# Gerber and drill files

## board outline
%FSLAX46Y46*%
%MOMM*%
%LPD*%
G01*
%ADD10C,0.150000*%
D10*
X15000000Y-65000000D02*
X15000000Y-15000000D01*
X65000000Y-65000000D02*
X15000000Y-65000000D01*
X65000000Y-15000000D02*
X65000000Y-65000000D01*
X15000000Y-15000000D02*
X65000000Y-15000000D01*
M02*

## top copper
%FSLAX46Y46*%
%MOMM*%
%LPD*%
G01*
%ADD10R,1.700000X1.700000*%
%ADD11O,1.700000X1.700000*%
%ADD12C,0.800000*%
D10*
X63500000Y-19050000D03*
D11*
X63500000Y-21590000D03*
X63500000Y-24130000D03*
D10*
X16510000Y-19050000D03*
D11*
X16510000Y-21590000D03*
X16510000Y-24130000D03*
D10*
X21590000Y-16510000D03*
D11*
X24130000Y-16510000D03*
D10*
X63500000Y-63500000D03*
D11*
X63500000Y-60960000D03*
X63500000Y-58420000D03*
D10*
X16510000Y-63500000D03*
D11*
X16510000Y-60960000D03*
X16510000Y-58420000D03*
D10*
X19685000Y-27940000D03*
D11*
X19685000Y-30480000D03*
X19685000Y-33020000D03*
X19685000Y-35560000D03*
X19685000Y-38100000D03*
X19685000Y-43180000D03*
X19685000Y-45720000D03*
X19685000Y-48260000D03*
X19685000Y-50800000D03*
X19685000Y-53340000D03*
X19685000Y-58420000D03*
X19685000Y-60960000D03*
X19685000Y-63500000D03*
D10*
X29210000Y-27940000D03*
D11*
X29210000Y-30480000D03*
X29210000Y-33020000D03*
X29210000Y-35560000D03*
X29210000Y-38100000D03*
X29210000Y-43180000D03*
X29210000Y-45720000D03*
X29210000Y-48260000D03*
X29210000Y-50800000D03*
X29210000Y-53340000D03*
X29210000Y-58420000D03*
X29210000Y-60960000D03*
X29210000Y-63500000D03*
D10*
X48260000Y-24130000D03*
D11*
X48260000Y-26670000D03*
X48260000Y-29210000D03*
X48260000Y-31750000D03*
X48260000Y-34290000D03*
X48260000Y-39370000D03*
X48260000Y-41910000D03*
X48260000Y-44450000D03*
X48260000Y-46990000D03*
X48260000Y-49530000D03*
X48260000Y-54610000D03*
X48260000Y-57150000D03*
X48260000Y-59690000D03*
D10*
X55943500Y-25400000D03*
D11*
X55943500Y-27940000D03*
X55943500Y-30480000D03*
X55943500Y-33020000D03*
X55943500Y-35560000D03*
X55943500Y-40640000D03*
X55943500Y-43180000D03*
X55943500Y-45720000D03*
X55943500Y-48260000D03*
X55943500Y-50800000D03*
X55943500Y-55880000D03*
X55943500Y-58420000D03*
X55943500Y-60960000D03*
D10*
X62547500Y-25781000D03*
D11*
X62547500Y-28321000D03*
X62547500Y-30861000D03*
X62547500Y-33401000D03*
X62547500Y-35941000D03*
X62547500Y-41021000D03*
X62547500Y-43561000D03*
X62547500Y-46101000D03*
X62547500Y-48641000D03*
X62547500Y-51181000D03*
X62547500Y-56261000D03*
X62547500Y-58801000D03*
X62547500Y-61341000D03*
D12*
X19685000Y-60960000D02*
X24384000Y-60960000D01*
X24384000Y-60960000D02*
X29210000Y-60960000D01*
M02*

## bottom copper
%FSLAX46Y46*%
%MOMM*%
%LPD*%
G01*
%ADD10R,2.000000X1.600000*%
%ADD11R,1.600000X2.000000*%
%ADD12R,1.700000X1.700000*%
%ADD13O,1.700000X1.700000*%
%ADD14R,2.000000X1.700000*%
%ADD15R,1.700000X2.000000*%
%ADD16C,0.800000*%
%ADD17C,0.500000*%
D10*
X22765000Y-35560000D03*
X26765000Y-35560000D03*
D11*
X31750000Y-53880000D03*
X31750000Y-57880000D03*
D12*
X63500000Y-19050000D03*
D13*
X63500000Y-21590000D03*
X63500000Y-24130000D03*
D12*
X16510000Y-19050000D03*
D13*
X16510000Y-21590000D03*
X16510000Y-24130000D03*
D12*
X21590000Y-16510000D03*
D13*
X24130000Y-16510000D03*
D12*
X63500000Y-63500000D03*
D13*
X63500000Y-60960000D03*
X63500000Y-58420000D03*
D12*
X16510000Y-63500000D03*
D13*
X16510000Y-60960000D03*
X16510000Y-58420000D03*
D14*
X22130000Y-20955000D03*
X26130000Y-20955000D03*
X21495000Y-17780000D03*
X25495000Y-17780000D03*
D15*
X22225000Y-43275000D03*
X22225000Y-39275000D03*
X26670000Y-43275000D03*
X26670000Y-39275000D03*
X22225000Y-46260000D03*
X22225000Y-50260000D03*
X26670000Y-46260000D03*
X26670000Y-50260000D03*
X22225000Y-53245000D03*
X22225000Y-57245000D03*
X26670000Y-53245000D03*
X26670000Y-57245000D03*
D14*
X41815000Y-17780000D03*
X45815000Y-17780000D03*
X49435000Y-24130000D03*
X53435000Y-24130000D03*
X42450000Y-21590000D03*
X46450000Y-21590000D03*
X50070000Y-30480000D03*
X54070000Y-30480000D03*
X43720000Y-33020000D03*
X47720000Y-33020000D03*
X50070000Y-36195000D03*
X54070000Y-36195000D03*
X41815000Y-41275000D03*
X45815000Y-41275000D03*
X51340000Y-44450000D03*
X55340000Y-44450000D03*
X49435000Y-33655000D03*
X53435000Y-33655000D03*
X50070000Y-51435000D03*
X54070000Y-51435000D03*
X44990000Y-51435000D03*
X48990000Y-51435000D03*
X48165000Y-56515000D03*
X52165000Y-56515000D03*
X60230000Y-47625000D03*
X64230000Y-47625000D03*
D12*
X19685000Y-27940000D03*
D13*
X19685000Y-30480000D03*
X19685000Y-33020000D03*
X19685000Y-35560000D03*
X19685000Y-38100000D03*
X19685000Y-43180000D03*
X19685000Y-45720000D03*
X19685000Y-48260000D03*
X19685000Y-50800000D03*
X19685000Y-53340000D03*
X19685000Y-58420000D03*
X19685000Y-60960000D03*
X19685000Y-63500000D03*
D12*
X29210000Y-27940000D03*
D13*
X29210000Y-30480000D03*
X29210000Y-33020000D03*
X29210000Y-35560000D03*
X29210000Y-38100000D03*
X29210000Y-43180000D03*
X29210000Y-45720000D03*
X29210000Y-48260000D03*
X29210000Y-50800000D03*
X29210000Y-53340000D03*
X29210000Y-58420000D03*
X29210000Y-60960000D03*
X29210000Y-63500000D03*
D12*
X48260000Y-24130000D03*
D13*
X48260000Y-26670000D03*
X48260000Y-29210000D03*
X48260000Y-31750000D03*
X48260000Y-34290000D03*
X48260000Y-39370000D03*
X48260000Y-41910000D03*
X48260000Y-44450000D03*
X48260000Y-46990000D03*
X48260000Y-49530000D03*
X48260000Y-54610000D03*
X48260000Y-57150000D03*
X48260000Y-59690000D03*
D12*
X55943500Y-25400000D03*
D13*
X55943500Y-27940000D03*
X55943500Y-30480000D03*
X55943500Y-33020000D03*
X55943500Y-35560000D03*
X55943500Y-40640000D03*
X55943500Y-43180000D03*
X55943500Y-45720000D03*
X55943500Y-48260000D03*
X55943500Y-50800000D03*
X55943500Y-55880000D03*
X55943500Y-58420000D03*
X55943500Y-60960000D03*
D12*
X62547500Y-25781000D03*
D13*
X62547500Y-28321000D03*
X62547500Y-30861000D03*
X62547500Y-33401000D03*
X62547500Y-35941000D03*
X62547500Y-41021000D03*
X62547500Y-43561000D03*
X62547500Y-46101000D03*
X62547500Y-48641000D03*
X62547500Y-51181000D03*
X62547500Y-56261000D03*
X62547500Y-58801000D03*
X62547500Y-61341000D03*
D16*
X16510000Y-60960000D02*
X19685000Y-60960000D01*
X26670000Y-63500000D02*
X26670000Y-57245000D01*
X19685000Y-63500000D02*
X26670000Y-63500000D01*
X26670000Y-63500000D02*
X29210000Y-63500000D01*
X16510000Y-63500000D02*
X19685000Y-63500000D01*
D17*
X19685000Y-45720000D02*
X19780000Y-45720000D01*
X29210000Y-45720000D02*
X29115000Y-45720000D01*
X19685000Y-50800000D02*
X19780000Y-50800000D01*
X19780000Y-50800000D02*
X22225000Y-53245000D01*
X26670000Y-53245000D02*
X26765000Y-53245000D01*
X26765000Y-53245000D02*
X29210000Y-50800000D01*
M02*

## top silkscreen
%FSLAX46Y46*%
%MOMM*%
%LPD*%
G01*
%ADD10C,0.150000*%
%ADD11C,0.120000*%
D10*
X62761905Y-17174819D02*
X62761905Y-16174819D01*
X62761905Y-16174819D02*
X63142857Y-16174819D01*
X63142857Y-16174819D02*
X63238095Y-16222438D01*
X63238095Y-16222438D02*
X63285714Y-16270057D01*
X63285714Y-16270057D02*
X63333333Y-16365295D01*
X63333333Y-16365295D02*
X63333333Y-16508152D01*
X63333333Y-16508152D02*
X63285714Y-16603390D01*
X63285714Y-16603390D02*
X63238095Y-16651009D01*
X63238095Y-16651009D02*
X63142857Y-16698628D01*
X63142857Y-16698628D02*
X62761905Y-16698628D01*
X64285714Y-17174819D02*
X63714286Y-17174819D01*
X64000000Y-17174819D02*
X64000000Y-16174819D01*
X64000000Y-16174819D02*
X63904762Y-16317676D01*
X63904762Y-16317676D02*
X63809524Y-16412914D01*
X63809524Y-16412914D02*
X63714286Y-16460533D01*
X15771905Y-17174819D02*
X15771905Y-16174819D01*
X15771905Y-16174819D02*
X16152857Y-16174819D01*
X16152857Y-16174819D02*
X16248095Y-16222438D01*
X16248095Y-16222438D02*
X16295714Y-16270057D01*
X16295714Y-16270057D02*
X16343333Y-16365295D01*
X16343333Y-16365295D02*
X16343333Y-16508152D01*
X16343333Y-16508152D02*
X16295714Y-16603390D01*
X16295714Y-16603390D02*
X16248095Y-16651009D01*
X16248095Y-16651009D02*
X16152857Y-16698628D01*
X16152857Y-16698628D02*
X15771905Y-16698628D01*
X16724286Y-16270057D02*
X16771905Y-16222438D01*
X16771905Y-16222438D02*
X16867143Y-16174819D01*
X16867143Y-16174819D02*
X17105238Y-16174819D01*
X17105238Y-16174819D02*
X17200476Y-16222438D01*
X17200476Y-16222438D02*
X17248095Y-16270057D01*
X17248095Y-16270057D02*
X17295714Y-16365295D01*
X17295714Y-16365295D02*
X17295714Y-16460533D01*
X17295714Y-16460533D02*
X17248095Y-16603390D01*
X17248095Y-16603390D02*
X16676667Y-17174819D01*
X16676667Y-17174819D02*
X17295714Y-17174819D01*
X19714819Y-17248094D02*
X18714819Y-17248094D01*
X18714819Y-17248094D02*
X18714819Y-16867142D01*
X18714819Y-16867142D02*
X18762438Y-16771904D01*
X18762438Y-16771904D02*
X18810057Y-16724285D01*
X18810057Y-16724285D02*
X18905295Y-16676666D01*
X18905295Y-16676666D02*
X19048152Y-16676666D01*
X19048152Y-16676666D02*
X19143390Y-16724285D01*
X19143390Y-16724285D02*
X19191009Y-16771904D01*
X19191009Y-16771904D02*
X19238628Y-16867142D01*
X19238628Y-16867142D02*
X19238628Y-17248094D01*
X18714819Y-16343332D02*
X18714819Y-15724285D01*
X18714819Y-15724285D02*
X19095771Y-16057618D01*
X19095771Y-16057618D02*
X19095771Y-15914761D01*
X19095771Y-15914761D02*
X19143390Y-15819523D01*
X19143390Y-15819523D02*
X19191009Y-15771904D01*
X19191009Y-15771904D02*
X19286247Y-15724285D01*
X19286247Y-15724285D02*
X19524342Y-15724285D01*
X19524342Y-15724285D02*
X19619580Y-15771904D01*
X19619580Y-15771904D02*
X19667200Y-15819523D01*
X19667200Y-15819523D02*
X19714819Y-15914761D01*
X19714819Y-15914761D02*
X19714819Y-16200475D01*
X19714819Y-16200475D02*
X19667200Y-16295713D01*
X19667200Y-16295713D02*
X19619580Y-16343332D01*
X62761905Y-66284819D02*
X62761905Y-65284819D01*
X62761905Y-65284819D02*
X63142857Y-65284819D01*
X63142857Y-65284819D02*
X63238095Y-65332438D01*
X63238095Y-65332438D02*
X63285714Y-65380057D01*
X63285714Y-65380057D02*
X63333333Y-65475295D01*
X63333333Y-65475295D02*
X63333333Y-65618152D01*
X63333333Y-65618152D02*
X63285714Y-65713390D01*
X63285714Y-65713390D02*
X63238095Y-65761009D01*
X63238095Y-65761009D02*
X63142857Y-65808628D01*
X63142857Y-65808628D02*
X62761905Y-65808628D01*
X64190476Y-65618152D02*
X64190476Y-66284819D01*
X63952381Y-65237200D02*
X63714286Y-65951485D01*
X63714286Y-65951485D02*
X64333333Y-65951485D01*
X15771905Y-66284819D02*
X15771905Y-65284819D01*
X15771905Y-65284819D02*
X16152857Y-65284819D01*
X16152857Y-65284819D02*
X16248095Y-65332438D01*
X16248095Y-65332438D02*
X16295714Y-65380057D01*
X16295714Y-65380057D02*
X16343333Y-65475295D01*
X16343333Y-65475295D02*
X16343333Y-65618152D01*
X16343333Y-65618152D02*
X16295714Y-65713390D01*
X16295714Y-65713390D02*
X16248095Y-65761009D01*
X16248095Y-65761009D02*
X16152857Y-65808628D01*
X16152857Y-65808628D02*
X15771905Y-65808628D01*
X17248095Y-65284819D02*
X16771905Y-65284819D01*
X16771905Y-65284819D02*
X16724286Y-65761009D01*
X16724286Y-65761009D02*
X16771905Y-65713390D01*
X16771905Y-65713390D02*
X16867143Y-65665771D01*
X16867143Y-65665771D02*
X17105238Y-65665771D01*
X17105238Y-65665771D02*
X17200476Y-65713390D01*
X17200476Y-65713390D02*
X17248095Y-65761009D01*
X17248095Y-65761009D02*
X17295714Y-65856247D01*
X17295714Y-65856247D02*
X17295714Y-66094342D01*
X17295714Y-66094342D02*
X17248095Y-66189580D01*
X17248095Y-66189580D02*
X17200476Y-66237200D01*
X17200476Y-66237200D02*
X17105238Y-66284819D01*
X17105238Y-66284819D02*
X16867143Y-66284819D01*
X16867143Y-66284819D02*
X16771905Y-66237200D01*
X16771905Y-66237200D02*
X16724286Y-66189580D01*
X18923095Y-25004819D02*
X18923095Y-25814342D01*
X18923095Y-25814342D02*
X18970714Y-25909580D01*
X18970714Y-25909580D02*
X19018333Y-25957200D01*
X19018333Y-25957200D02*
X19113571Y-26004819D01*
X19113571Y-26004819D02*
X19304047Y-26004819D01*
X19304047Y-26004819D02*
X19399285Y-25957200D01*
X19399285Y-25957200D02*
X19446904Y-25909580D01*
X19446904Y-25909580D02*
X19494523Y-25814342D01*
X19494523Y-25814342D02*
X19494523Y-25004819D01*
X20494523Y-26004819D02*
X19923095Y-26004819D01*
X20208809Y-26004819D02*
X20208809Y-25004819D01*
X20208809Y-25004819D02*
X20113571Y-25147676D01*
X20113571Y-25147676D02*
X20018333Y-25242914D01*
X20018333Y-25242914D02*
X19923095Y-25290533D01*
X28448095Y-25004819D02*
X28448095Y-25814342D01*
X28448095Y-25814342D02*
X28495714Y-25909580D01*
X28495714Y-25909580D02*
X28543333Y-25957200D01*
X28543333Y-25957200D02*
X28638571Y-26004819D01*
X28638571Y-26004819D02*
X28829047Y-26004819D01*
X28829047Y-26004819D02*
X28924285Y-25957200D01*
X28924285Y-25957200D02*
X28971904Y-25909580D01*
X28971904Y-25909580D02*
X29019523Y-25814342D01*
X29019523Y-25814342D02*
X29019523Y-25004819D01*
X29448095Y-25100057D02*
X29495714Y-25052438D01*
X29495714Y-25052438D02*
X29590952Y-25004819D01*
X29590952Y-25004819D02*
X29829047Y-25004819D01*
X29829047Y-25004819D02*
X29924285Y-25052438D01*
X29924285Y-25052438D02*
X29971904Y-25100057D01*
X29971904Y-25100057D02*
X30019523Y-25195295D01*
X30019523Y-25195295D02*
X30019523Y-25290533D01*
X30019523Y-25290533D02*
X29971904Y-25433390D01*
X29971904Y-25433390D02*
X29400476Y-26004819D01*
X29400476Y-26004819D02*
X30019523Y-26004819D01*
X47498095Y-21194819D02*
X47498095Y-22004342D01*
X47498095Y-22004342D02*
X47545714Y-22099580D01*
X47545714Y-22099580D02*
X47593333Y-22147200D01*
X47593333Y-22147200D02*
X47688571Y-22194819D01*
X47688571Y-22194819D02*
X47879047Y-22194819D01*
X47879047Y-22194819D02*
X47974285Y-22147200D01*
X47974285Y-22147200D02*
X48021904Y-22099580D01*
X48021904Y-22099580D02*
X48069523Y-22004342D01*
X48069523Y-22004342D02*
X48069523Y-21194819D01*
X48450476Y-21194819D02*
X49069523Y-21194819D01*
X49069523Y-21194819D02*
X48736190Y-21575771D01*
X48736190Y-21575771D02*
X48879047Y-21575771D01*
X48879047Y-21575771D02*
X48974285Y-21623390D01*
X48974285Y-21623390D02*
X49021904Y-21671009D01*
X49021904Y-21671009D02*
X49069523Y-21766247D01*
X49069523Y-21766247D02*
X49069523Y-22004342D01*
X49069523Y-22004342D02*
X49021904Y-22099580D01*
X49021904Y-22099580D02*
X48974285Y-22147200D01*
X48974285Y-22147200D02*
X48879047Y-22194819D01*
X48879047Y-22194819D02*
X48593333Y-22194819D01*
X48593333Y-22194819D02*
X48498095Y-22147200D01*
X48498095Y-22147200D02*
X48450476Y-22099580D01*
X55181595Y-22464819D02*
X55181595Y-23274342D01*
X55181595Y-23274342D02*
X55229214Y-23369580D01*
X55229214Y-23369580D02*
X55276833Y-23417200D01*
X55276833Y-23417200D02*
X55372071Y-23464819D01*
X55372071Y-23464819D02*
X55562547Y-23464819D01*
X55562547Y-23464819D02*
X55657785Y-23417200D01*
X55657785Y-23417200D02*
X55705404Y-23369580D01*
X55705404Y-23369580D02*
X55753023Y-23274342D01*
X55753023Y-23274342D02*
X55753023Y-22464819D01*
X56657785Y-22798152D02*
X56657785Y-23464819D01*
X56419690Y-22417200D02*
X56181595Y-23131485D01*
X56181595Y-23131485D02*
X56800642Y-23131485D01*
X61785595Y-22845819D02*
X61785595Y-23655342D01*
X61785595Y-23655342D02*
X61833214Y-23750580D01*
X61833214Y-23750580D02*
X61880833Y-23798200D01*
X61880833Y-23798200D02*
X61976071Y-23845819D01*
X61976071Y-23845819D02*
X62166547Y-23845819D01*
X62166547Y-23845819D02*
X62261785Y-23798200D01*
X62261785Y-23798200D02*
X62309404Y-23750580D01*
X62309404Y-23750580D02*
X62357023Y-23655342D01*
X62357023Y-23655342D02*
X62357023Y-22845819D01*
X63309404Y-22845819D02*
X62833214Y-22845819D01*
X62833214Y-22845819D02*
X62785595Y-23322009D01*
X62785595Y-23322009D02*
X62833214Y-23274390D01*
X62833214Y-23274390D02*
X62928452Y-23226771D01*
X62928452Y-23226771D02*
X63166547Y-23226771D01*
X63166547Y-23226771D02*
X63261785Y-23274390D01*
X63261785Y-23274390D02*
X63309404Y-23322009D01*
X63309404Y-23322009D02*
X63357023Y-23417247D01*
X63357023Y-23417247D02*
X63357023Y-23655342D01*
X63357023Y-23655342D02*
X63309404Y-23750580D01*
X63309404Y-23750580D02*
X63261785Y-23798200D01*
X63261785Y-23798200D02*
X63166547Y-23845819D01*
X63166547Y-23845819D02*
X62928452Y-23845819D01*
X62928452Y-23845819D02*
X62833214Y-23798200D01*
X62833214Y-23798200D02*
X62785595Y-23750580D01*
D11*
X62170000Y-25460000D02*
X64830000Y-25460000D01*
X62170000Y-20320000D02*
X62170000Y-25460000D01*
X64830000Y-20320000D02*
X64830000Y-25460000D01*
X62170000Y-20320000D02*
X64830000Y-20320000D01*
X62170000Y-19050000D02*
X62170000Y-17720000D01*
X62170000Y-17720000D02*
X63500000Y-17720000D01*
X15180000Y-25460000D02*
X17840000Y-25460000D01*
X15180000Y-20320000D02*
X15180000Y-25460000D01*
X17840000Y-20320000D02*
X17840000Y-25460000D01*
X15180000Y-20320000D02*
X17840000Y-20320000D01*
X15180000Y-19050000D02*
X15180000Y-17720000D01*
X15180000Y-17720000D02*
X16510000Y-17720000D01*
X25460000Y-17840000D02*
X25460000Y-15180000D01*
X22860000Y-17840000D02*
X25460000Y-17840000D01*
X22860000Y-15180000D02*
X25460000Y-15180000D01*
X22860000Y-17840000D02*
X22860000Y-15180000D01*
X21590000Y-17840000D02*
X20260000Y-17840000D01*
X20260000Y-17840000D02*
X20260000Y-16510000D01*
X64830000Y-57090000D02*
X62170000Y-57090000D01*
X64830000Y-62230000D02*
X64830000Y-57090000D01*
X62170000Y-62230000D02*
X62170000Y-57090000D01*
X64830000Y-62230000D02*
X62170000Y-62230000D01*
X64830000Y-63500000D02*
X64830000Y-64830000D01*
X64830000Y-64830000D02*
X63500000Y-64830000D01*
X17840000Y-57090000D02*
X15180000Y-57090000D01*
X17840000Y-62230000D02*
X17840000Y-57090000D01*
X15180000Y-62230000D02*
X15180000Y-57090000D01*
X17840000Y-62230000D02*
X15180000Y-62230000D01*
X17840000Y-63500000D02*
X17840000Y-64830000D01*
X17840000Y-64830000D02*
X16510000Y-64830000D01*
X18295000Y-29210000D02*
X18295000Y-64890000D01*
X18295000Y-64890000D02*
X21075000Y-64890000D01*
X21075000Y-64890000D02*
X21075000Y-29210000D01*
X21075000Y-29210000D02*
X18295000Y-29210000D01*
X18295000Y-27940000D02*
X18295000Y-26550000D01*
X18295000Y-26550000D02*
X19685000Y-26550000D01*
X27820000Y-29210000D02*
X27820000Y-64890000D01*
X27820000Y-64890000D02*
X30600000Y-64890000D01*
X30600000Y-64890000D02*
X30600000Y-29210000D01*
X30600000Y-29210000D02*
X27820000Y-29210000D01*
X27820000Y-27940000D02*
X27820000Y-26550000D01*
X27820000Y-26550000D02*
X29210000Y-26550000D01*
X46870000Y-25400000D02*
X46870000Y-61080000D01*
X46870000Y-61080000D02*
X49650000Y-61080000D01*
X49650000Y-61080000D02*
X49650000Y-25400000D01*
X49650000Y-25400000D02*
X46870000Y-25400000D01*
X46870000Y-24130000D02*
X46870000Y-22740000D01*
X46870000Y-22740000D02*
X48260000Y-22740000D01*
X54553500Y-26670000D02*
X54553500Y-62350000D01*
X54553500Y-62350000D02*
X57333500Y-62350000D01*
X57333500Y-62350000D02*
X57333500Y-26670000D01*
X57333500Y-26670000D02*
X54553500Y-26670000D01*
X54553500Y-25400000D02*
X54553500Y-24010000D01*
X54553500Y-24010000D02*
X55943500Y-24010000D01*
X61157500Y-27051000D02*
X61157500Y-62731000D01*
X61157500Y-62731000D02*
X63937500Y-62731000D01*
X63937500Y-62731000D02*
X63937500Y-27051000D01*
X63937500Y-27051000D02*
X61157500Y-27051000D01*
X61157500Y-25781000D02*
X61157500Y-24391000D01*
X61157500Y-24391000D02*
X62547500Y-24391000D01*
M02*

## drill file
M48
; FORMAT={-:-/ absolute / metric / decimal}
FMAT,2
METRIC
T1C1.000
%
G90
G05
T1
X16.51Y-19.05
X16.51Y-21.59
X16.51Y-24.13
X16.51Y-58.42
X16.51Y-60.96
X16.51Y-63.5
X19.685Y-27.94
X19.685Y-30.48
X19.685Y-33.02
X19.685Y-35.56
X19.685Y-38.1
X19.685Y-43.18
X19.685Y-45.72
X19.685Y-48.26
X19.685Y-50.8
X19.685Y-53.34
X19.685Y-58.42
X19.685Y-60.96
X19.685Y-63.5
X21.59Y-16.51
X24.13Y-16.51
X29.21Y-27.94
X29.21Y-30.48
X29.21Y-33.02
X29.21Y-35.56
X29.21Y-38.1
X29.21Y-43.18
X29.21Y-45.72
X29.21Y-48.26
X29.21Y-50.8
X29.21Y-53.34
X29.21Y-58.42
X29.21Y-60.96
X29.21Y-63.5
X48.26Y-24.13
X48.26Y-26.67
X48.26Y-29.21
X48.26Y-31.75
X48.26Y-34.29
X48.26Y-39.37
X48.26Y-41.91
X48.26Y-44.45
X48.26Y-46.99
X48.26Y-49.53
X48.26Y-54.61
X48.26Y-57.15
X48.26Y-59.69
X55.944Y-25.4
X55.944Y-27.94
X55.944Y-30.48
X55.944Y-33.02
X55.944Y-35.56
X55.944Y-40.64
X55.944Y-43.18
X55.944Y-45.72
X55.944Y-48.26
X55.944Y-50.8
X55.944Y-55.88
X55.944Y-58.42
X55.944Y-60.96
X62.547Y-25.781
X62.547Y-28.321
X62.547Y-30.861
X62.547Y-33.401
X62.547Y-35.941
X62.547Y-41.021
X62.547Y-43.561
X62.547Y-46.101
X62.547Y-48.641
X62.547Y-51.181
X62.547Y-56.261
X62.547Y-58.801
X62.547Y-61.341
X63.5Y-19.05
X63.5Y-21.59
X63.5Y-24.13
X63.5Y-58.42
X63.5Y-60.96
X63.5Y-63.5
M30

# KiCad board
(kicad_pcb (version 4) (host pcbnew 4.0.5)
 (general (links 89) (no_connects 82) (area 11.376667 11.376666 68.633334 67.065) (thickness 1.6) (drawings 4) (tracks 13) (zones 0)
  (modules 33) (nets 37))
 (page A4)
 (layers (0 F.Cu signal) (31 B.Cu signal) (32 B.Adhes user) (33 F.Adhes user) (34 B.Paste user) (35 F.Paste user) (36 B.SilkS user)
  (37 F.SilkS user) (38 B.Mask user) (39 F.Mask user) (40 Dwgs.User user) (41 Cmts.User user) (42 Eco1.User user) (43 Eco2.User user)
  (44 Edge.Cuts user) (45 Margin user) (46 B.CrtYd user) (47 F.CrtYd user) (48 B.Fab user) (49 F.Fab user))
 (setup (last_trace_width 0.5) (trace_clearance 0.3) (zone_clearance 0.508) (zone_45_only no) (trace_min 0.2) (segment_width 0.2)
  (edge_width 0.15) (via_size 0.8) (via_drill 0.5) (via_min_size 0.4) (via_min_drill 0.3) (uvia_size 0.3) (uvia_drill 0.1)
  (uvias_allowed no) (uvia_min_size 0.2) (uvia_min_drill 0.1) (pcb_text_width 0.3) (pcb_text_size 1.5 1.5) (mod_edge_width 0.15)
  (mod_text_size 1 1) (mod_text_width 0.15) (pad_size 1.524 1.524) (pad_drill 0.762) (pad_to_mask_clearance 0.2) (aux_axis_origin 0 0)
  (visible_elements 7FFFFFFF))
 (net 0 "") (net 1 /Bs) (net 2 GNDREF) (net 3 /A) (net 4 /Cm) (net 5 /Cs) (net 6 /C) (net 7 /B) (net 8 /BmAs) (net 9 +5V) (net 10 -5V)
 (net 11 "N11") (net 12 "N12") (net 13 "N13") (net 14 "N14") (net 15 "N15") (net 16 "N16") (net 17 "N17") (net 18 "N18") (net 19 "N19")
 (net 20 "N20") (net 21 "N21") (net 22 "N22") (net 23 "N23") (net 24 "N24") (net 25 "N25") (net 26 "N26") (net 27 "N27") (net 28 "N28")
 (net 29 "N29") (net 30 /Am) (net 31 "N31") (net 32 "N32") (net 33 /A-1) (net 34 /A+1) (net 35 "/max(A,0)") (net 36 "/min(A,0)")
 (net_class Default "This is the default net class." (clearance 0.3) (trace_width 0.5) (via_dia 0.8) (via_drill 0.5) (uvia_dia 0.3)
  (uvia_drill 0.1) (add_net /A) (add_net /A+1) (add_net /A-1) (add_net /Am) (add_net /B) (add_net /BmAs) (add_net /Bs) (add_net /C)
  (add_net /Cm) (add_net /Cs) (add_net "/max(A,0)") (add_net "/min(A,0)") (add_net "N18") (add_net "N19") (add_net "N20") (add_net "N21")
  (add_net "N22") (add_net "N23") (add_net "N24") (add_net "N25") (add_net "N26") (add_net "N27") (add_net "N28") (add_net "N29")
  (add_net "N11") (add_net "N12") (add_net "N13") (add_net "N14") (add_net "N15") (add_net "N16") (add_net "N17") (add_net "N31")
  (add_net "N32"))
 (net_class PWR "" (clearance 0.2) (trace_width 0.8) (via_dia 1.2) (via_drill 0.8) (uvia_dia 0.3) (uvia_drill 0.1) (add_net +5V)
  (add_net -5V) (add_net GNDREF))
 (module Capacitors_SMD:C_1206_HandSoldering (layer B.Cu) (at 24.765 35.56)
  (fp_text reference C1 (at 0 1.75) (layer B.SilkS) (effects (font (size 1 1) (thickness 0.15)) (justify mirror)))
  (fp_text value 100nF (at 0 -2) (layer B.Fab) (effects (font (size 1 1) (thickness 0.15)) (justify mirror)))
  (pad 1 smd rect (at -2 0) (size 2 1.6) (layers B.Cu B.Paste B.Mask) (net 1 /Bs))
  (pad 2 smd rect (at 2 0) (size 2 1.6) (layers B.Cu B.Paste B.Mask) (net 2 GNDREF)))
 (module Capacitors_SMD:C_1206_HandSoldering (layer B.Cu) (at 31.75 55.88 270)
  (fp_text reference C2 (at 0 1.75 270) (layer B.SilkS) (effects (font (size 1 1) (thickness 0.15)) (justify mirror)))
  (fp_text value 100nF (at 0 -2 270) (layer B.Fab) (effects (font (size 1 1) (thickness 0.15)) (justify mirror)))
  (pad 1 smd rect (at -2 0 270) (size 2 1.6) (layers B.Cu B.Paste B.Mask) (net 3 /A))
  (pad 2 smd rect (at 2 0 270) (size 2 1.6) (layers B.Cu B.Paste B.Mask) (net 2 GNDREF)))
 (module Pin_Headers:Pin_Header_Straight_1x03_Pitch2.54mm (layer F.Cu) (at 63.5 19.05)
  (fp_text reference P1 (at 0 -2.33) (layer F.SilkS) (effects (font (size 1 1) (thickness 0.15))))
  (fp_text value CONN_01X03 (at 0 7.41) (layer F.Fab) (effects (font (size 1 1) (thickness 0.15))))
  (fp_line (start -1.33 6.41) (end 1.33 6.41) (layer F.SilkS) (width 0.12))
  (fp_line (start -1.33 1.27) (end -1.33 6.41) (layer F.SilkS) (width 0.12))
  (fp_line (start 1.33 1.27) (end 1.33 6.41) (layer F.SilkS) (width 0.12))
  (fp_line (start -1.33 1.27) (end 1.33 1.27) (layer F.SilkS) (width 0.12))
  (fp_line (start -1.33 0) (end -1.33 -1.33) (layer F.SilkS) (width 0.12))
  (fp_line (start -1.33 -1.33) (end 0 -1.33) (layer F.SilkS) (width 0.12))
  (pad 1 thru_hole rect (at 0 0) (size 1.7 1.7) (drill 1) (layers *.Cu *.Mask) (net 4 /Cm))
  (pad 2 thru_hole oval (at 0 2.54) (size 1.7 1.7) (drill 1) (layers *.Cu *.Mask) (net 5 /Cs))
  (pad 3 thru_hole oval (at 0 5.08) (size 1.7 1.7) (drill 1) (layers *.Cu *.Mask) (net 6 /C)))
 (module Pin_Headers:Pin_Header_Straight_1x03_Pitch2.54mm (layer F.Cu) (at 16.51 19.05)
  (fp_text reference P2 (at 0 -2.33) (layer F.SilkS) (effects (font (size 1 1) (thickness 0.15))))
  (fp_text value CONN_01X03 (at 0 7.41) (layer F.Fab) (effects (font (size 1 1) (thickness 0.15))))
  (fp_line (start -1.33 6.41) (end 1.33 6.41) (layer F.SilkS) (width 0.12))
  (fp_line (start -1.33 1.27) (end -1.33 6.41) (layer F.SilkS) (width 0.12))
  (fp_line (start 1.33 1.27) (end 1.33 6.41) (layer F.SilkS) (width 0.12))
  (fp_line (start -1.33 1.27) (end 1.33 1.27) (layer F.SilkS) (width 0.12))
  (fp_line (start -1.33 0) (end -1.33 -1.33) (layer F.SilkS) (width 0.12))
  (fp_line (start -1.33 -1.33) (end 0 -1.33) (layer F.SilkS) (width 0.12))
  (pad 1 thru_hole rect (at 0 0) (size 1.7 1.7) (drill 1) (layers *.Cu *.Mask) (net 4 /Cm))
  (pad 2 thru_hole oval (at 0 2.54) (size 1.7 1.7) (drill 1) (layers *.Cu *.Mask) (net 5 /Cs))
  (pad 3 thru_hole oval (at 0 5.08) (size 1.7 1.7) (drill 1) (layers *.Cu *.Mask) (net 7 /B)))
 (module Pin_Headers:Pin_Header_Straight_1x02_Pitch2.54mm (layer F.Cu) (at 21.59 16.51 90)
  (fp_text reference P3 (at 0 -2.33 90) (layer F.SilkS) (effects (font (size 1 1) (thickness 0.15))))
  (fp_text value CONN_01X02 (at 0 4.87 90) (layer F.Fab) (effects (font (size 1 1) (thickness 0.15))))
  (fp_line (start -1.33 3.87) (end 1.33 3.87) (layer F.SilkS) (width 0.12))
  (fp_line (start -1.33 1.27) (end -1.33 3.87) (layer F.SilkS) (width 0.12))
  (fp_line (start 1.33 1.27) (end 1.33 3.87) (layer F.SilkS) (width 0.12))
  (fp_line (start -1.33 1.27) (end 1.33 1.27) (layer F.SilkS) (width 0.12))
  (fp_line (start -1.33 0) (end -1.33 -1.33) (layer F.SilkS) (width 0.12))
  (fp_line (start -1.33 -1.33) (end 0 -1.33) (layer F.SilkS) (width 0.12))
  (pad 1 thru_hole rect (at 0 0 90) (size 1.7 1.7) (drill 1) (layers *.Cu *.Mask) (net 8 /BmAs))
  (pad 2 thru_hole oval (at 0 2.54 90) (size 1.7 1.7) (drill 1) (layers *.Cu *.Mask) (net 3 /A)))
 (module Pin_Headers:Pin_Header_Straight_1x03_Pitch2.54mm (layer F.Cu) (at 63.5 63.5 180)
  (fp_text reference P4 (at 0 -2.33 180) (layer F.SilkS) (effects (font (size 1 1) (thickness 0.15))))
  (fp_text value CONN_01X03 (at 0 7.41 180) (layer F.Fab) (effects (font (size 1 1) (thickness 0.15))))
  (fp_line (start -1.33 6.41) (end 1.33 6.41) (layer F.SilkS) (width 0.12))
  (fp_line (start -1.33 1.27) (end -1.33 6.41) (layer F.SilkS) (width 0.12))
  (fp_line (start 1.33 1.27) (end 1.33 6.41) (layer F.SilkS) (width 0.12))
  (fp_line (start -1.33 1.27) (end 1.33 1.27) (layer F.SilkS) (width 0.12))
  (fp_line (start -1.33 0) (end -1.33 -1.33) (layer F.SilkS) (width 0.12))
  (fp_line (start -1.33 -1.33) (end 0 -1.33) (layer F.SilkS) (width 0.12))
  (pad 1 thru_hole rect (at 0 0 180) (size 1.7 1.7) (drill 1) (layers *.Cu *.Mask) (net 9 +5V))
  (pad 2 thru_hole oval (at 0 2.54 180) (size 1.7 1.7) (drill 1) (layers *.Cu *.Mask) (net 2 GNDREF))
  (pad 3 thru_hole oval (at 0 5.08 180) (size 1.7 1.7) (drill 1) (layers *.Cu *.Mask) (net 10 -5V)))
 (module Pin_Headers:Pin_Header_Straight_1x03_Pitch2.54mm (layer F.Cu) (at 16.51 63.5 180)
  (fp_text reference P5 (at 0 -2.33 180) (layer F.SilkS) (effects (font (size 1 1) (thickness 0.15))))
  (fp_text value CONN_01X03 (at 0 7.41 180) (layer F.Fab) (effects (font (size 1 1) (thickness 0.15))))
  (fp_line (start -1.33 6.41) (end 1.33 6.41) (layer F.SilkS) (width 0.12))
  (fp_line (start -1.33 1.27) (end -1.33 6.41) (layer F.SilkS) (width 0.12))
  (fp_line (start 1.33 1.27) (end 1.33 6.41) (layer F.SilkS) (width 0.12))
  (fp_line (start -1.33 1.27) (end 1.33 1.27) (layer F.SilkS) (width 0.12))
  (fp_line (start -1.33 0) (end -1.33 -1.33) (layer F.SilkS) (width 0.12))
  (fp_line (start -1.33 -1.33) (end 0 -1.33) (layer F.SilkS) (width 0.12))
  (pad 1 thru_hole rect (at 0 0 180) (size 1.7 1.7) (drill 1) (layers *.Cu *.Mask) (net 9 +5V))
  (pad 2 thru_hole oval (at 0 2.54 180) (size 1.7 1.7) (drill 1) (layers *.Cu *.Mask) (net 2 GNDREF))
  (pad 3 thru_hole oval (at 0 5.08 180) (size 1.7 1.7) (drill 1) (layers *.Cu *.Mask) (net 10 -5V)))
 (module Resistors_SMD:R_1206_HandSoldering (layer B.Cu) (at 24.13 20.955)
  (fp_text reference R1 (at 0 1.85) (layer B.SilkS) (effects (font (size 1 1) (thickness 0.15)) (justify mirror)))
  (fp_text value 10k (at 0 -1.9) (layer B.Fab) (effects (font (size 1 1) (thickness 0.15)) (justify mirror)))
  (pad 1 smd rect (at -2 0) (size 2 1.7) (layers B.Cu B.Paste B.Mask) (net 5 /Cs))
  (pad 2 smd rect (at 2 0) (size 2 1.7) (layers B.Cu B.Paste B.Mask) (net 2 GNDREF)))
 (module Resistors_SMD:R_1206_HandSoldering (layer B.Cu) (at 23.495 17.78)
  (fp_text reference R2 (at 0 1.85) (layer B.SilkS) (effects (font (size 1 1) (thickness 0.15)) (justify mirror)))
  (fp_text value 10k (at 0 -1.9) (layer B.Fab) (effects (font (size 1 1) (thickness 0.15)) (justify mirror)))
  (pad 1 smd rect (at -2 0) (size 2 1.7) (layers B.Cu B.Paste B.Mask) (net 4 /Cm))
  (pad 2 smd rect (at 2 0) (size 2 1.7) (layers B.Cu B.Paste B.Mask) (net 2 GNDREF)))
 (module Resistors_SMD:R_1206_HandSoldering (layer B.Cu) (at 22.225 41.275 90)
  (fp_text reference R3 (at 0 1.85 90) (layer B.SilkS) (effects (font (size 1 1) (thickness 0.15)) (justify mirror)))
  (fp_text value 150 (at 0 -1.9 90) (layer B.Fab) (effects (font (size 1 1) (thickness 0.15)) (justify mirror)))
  (pad 1 smd rect (at -2 0 90) (size 2 1.7) (layers B.Cu B.Paste B.Mask) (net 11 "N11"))
  (pad 2 smd rect (at 2 0 90) (size 2 1.7) (layers B.Cu B.Paste B.Mask) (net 10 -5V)))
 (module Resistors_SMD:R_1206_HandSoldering (layer B.Cu) (at 26.67 41.275 90)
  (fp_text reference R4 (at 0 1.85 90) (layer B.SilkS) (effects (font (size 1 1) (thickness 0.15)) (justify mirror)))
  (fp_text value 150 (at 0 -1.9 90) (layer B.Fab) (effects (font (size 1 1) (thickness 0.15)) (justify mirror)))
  (pad 1 smd rect (at -2 0 90) (size 2 1.7) (layers B.Cu B.Paste B.Mask) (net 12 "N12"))
  (pad 2 smd rect (at 2 0 90) (size 2 1.7) (layers B.Cu B.Paste B.Mask) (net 10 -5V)))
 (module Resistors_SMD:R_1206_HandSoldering (layer B.Cu) (at 22.225 48.26 270)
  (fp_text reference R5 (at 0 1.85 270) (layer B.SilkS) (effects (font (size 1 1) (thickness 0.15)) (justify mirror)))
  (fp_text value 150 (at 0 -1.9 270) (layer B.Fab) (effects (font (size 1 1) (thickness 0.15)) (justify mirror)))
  (pad 1 smd rect (at -2 0 270) (size 2 1.7) (layers B.Cu B.Paste B.Mask) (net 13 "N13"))
  (pad 2 smd rect (at 2 0 270) (size 2 1.7) (layers B.Cu B.Paste B.Mask) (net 2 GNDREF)))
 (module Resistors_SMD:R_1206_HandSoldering (layer B.Cu) (at 26.67 48.26 270)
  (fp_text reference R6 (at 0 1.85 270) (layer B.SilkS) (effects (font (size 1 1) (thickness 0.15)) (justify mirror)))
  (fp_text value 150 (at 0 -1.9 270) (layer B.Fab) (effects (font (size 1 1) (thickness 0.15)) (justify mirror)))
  (pad 1 smd rect (at -2 0 270) (size 2 1.7) (layers B.Cu B.Paste B.Mask) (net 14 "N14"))
  (pad 2 smd rect (at 2 0 270) (size 2 1.7) (layers B.Cu B.Paste B.Mask) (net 2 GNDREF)))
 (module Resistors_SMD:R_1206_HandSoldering (layer B.Cu) (at 22.225 55.245 270)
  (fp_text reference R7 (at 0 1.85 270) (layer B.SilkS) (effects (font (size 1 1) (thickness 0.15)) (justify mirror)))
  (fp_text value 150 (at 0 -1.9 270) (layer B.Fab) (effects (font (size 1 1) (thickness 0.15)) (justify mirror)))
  (pad 1 smd rect (at -2 0 270) (size 2 1.7) (layers B.Cu B.Paste B.Mask) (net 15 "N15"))
  (pad 2 smd rect (at 2 0 270) (size 2 1.7) (layers B.Cu B.Paste B.Mask) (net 9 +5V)))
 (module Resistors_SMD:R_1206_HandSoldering (layer B.Cu) (at 26.67 55.245 270)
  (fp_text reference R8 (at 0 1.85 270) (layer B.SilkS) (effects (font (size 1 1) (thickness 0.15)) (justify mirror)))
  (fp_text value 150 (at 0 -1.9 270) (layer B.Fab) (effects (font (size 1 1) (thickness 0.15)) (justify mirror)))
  (pad 1 smd rect (at -2 0 270) (size 2 1.7) (layers B.Cu B.Paste B.Mask) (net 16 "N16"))
  (pad 2 smd rect (at 2 0 270) (size 2 1.7) (layers B.Cu B.Paste B.Mask) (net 9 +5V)))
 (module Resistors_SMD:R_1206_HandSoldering (layer B.Cu) (at 43.815 17.78)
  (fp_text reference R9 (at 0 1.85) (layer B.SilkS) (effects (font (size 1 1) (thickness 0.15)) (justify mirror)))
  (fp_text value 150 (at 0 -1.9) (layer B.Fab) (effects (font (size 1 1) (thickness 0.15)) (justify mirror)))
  (pad 1 smd rect (at -2 0) (size 2 1.7) (layers B.Cu B.Paste B.Mask) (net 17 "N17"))
  (pad 2 smd rect (at 2 0) (size 2 1.7) (layers B.Cu B.Paste B.Mask) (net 9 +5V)))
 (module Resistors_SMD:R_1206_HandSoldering (layer B.Cu) (at 51.435 24.13)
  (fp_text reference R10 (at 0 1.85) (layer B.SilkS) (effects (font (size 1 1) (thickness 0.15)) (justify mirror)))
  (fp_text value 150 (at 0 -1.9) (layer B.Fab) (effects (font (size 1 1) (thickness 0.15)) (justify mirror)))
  (pad 1 smd rect (at -2 0) (size 2 1.7) (layers B.Cu B.Paste B.Mask) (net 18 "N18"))
  (pad 2 smd rect (at 2 0) (size 2 1.7) (layers B.Cu B.Paste B.Mask) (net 2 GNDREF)))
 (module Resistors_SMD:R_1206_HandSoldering (layer B.Cu) (at 44.45 21.59)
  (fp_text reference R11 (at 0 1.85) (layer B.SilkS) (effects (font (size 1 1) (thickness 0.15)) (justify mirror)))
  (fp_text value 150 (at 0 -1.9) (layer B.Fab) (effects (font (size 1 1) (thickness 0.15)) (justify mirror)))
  (pad 1 smd rect (at -2 0) (size 2 1.7) (layers B.Cu B.Paste B.Mask) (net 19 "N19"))
  (pad 2 smd rect (at 2 0) (size 2 1.7) (layers B.Cu B.Paste B.Mask) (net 10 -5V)))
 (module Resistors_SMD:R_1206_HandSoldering (layer B.Cu) (at 52.07 30.48)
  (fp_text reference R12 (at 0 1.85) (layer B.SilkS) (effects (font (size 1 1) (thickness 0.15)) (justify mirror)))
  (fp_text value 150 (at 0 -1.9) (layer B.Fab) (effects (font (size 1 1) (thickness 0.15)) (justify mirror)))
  (pad 1 smd rect (at -2 0) (size 2 1.7) (layers B.Cu B.Paste B.Mask) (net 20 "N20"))
  (pad 2 smd rect (at 2 0) (size 2 1.7) (layers B.Cu B.Paste B.Mask) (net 2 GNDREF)))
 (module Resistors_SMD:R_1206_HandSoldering (layer B.Cu) (at 45.72 33.02)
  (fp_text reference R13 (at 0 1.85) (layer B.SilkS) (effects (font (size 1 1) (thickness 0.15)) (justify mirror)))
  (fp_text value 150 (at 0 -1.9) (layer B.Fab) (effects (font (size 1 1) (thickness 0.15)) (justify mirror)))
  (pad 1 smd rect (at -2 0) (size 2 1.7) (layers B.Cu B.Paste B.Mask) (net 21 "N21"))
  (pad 2 smd rect (at 2 0) (size 2 1.7) (layers B.Cu B.Paste B.Mask) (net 2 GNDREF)))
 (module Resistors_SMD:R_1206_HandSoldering (layer B.Cu) (at 52.07 36.195)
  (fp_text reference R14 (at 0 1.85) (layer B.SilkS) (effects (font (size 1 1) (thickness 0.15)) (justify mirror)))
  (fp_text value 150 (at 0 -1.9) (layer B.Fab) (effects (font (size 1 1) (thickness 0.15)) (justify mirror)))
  (pad 1 smd rect (at -2 0) (size 2 1.7) (layers B.Cu B.Paste B.Mask) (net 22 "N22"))
  (pad 2 smd rect (at 2 0) (size 2 1.7) (layers B.Cu B.Paste B.Mask) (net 9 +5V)))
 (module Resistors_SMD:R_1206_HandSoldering (layer B.Cu) (at 43.815 41.275)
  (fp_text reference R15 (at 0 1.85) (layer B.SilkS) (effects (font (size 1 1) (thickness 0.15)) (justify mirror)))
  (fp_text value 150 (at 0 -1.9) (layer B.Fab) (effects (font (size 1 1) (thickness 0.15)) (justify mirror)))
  (pad 1 smd rect (at -2 0) (size 2 1.7) (layers B.Cu B.Paste B.Mask) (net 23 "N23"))
  (pad 2 smd rect (at 2 0) (size 2 1.7) (layers B.Cu B.Paste B.Mask) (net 2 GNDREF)))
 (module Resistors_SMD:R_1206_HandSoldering (layer B.Cu) (at 53.34 44.45)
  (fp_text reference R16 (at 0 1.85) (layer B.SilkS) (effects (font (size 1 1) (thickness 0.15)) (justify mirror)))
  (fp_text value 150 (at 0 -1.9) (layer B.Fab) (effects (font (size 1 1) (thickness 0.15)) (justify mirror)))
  (pad 1 smd rect (at -2 0) (size 2 1.7) (layers B.Cu B.Paste B.Mask) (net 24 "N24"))
  (pad 2 smd rect (at 2 0) (size 2 1.7) (layers B.Cu B.Paste B.Mask) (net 10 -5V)))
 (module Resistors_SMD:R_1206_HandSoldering (layer B.Cu) (at 51.435 33.655)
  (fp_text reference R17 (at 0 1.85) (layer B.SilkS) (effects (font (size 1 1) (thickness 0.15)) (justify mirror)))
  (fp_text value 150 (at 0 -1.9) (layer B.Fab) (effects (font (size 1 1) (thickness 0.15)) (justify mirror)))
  (pad 1 smd rect (at -2 0) (size 2 1.7) (layers B.Cu B.Paste B.Mask) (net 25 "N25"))
  (pad 2 smd rect (at 2 0) (size 2 1.7) (layers B.Cu B.Paste B.Mask) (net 9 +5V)))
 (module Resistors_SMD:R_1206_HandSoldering (layer B.Cu) (at 52.07 51.435)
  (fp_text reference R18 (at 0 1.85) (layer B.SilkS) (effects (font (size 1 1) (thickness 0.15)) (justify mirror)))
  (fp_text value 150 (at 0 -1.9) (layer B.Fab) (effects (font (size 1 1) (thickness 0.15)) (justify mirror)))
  (pad 1 smd rect (at -2 0) (size 2 1.7) (layers B.Cu B.Paste B.Mask) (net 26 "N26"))
  (pad 2 smd rect (at 2 0) (size 2 1.7) (layers B.Cu B.Paste B.Mask) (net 2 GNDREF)))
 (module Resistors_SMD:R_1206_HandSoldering (layer B.Cu) (at 46.99 51.435)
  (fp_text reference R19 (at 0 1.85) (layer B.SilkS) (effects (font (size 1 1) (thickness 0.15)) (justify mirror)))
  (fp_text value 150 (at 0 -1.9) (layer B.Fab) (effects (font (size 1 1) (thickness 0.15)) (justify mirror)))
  (pad 1 smd rect (at -2 0) (size 2 1.7) (layers B.Cu B.Paste B.Mask) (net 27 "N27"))
  (pad 2 smd rect (at 2 0) (size 2 1.7) (layers B.Cu B.Paste B.Mask) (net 10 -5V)))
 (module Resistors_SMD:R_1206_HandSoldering (layer B.Cu) (at 50.165 56.515)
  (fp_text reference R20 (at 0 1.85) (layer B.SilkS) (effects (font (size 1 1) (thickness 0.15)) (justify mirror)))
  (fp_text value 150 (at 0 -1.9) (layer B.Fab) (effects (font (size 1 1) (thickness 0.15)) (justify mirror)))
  (pad 1 smd rect (at -2 0) (size 2 1.7) (layers B.Cu B.Paste B.Mask) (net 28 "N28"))
  (pad 2 smd rect (at 2 0) (size 2 1.7) (layers B.Cu B.Paste B.Mask) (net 2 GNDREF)))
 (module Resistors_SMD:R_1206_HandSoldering (layer B.Cu) (at 62.23 47.625)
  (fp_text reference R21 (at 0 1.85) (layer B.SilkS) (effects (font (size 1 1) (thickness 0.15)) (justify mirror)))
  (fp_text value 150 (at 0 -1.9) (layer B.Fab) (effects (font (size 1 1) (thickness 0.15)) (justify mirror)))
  (pad 1 smd rect (at -2 0) (size 2 1.7) (layers B.Cu B.Paste B.Mask) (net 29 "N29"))
  (pad 2 smd rect (at 2 0) (size 2 1.7) (layers B.Cu B.Paste B.Mask) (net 2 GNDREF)))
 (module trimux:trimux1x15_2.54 (layer F.Cu) (at 19.685 27.94)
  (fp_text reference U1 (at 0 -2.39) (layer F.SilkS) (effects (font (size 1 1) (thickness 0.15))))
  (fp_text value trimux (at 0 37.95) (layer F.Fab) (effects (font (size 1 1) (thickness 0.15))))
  (fp_line (start -1.39 1.27) (end -1.39 36.95) (layer F.SilkS) (width 0.12))
  (fp_line (start -1.39 36.95) (end 1.39 36.95) (layer F.SilkS) (width 0.12))
  (fp_line (start 1.39 36.95) (end 1.39 1.27) (layer F.SilkS) (width 0.12))
  (fp_line (start 1.39 1.27) (end -1.39 1.27) (layer F.SilkS) (width 0.12))
  (fp_line (start -1.39 0) (end -1.39 -1.39) (layer F.SilkS) (width 0.12))
  (fp_line (start -1.39 -1.39) (end 0 -1.39) (layer F.SilkS) (width 0.12))
  (pad 1 thru_hole rect (at 0 0) (size 1.7 1.7) (drill 1) (layers *.Cu *.Mask) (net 4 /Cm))
  (pad 2 thru_hole oval (at 0 2.54) (size 1.7 1.7) (drill 1) (layers *.Cu *.Mask) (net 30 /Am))
  (pad 3 thru_hole oval (at 0 5.08) (size 1.7 1.7) (drill 1) (layers *.Cu *.Mask) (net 1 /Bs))
  (pad 4 thru_hole oval (at 0 7.62) (size 1.7 1.7) (drill 1) (layers *.Cu *.Mask) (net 8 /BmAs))
  (pad 5 thru_hole oval (at 0 10.16) (size 1.7 1.7) (drill 1) (layers *.Cu *.Mask) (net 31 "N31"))
  (pad 7 thru_hole oval (at 0 15.24) (size 1.7 1.7) (drill 1) (layers *.Cu *.Mask) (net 31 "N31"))
  (pad 8 thru_hole oval (at 0 17.78) (size 1.7 1.7) (drill 1) (layers *.Cu *.Mask) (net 11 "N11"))
  (pad 9 thru_hole oval (at 0 20.32) (size 1.7 1.7) (drill 1) (layers *.Cu *.Mask) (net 13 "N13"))
  (pad 10 thru_hole oval (at 0 22.86) (size 1.7 1.7) (drill 1) (layers *.Cu *.Mask) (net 15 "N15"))
  (pad 11 thru_hole oval (at 0 25.4) (size 1.7 1.7) (drill 1) (layers *.Cu *.Mask) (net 1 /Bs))
  (pad 13 thru_hole oval (at 0 30.48) (size 1.7 1.7) (drill 1) (layers *.Cu *.Mask) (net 10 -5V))
  (pad 14 thru_hole oval (at 0 33.02) (size 1.7 1.7) (drill 1) (layers *.Cu *.Mask) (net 2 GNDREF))
  (pad 15 thru_hole oval (at 0 35.56) (size 1.7 1.7) (drill 1) (layers *.Cu *.Mask) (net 9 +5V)))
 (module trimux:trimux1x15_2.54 (layer F.Cu) (at 29.21 27.94)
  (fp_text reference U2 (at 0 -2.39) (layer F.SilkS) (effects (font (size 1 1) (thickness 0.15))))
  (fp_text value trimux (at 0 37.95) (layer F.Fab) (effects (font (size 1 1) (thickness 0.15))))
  (fp_line (start -1.39 1.27) (end -1.39 36.95) (layer F.SilkS) (width 0.12))
  (fp_line (start -1.39 36.95) (end 1.39 36.95) (layer F.SilkS) (width 0.12))
  (fp_line (start 1.39 36.95) (end 1.39 1.27) (layer F.SilkS) (width 0.12))
  (fp_line (start 1.39 1.27) (end -1.39 1.27) (layer F.SilkS) (width 0.12))
  (fp_line (start -1.39 0) (end -1.39 -1.39) (layer F.SilkS) (width 0.12))
  (fp_line (start -1.39 -1.39) (end 0 -1.39) (layer F.SilkS) (width 0.12))
  (pad 1 thru_hole rect (at 0 0) (size 1.7 1.7) (drill 1) (layers *.Cu *.Mask) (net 5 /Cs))
  (pad 2 thru_hole oval (at 0 2.54) (size 1.7 1.7) (drill 1) (layers *.Cu *.Mask) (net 8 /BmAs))
  (pad 3 thru_hole oval (at 0 5.08) (size 1.7 1.7) (drill 1) (layers *.Cu *.Mask) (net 3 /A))
  (pad 4 thru_hole oval (at 0 7.62) (size 1.7 1.7) (drill 1) (layers *.Cu *.Mask) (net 1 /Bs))
  (pad 5 thru_hole oval (at 0 10.16) (size 1.7 1.7) (drill 1) (layers *.Cu *.Mask) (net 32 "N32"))
  (pad 7 thru_hole oval (at 0 15.24) (size 1.7 1.7) (drill 1) (layers *.Cu *.Mask) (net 32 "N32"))
  (pad 8 thru_hole oval (at 0 17.78) (size 1.7 1.7) (drill 1) (layers *.Cu *.Mask) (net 12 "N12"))
  (pad 9 thru_hole oval (at 0 20.32) (size 1.7 1.7) (drill 1) (layers *.Cu *.Mask) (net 14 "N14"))
  (pad 10 thru_hole oval (at 0 22.86) (size 1.7 1.7) (drill 1) (layers *.Cu *.Mask) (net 16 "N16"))
  (pad 11 thru_hole oval (at 0 25.4) (size 1.7 1.7) (drill 1) (layers *.Cu *.Mask) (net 3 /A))
  (pad 13 thru_hole oval (at 0 30.48) (size 1.7 1.7) (drill 1) (layers *.Cu *.Mask) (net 10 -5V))
  (pad 14 thru_hole oval (at 0 33.02) (size 1.7 1.7) (drill 1) (layers *.Cu *.Mask) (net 2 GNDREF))
  (pad 15 thru_hole oval (at 0 35.56) (size 1.7 1.7) (drill 1) (layers *.Cu *.Mask) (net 9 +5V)))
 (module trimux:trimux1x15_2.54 (layer F.Cu) (at 48.26 24.13)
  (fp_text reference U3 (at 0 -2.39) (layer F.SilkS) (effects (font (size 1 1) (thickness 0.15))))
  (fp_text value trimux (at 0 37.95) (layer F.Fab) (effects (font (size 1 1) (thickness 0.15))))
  (fp_line (start -1.39 1.27) (end -1.39 36.95) (layer F.SilkS) (width 0.12))
  (fp_line (start -1.39 36.95) (end 1.39 36.95) (layer F.SilkS) (width 0.12))
  (fp_line (start 1.39 36.95) (end 1.39 1.27) (layer F.SilkS) (width 0.12))
  (fp_line (start 1.39 1.27) (end -1.39 1.27) (layer F.SilkS) (width 0.12))
  (fp_line (start -1.39 0) (end -1.39 -1.39) (layer F.SilkS) (width 0.12))
  (fp_line (start -1.39 -1.39) (end 0 -1.39) (layer F.SilkS) (width 0.12))
  (pad 1 thru_hole rect (at 0 0) (size 1.7 1.7) (drill 1) (layers *.Cu *.Mask) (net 3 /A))
  (pad 2 thru_hole oval (at 0 2.54) (size 1.7 1.7) (drill 1) (layers *.Cu *.Mask) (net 17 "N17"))
  (pad 3 thru_hole oval (at 0 5.08) (size 1.7 1.7) (drill 1) (layers *.Cu *.Mask) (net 19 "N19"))
  (pad 4 thru_hole oval (at 0 7.62) (size 1.7 1.7) (drill 1) (layers *.Cu *.Mask) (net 21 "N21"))
  (pad 5 thru_hole oval (at 0 10.16) (size 1.7 1.7) (drill 1) (layers *.Cu *.Mask) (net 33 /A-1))
  (pad 7 thru_hole oval (at 0 15.24) (size 1.7 1.7) (drill 1) (layers *.Cu *.Mask) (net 3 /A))
  (pad 8 thru_hole oval (at 0 17.78) (size 1.7 1.7) (drill 1) (layers *.Cu *.Mask) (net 23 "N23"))
  (pad 9 thru_hole oval (at 0 20.32) (size 1.7 1.7) (drill 1) (layers *.Cu *.Mask) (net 25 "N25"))
  (pad 10 thru_hole oval (at 0 22.86) (size 1.7 1.7) (drill 1) (layers *.Cu *.Mask) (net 27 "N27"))
  (pad 11 thru_hole oval (at 0 25.4) (size 1.7 1.7) (drill 1) (layers *.Cu *.Mask) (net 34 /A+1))
  (pad 13 thru_hole oval (at 0 30.48) (size 1.7 1.7) (drill 1) (layers *.Cu *.Mask) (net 10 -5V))
  (pad 14 thru_hole oval (at 0 33.02) (size 1.7 1.7) (drill 1) (layers *.Cu *.Mask) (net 2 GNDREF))
  (pad 15 thru_hole oval (at 0 35.56) (size 1.7 1.7) (drill 1) (layers *.Cu *.Mask) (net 9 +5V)))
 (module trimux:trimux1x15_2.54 (layer F.Cu) (at 55.9435 25.4)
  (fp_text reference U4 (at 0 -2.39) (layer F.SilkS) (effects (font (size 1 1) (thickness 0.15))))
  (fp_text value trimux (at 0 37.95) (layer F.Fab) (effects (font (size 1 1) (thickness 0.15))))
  (fp_line (start -1.39 1.27) (end -1.39 36.95) (layer F.SilkS) (width 0.12))
  (fp_line (start -1.39 36.95) (end 1.39 36.95) (layer F.SilkS) (width 0.12))
  (fp_line (start 1.39 36.95) (end 1.39 1.27) (layer F.SilkS) (width 0.12))
  (fp_line (start 1.39 1.27) (end -1.39 1.27) (layer F.SilkS) (width 0.12))
  (fp_line (start -1.39 0) (end -1.39 -1.39) (layer F.SilkS) (width 0.12))
  (fp_line (start -1.39 -1.39) (end 0 -1.39) (layer F.SilkS) (width 0.12))
  (pad 1 thru_hole rect (at 0 0) (size 1.7 1.7) (drill 1) (layers *.Cu *.Mask) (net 3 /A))
  (pad 2 thru_hole oval (at 0 2.54) (size 1.7 1.7) (drill 1) (layers *.Cu *.Mask) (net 18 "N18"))
  (pad 3 thru_hole oval (at 0 5.08) (size 1.7 1.7) (drill 1) (layers *.Cu *.Mask) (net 20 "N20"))
  (pad 4 thru_hole oval (at 0 7.62) (size 1.7 1.7) (drill 1) (layers *.Cu *.Mask) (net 22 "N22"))
  (pad 5 thru_hole oval (at 0 10.16) (size 1.7 1.7) (drill 1) (layers *.Cu *.Mask) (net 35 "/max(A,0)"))
  (pad 7 thru_hole oval (at 0 15.24) (size 1.7 1.7) (drill 1) (layers *.Cu *.Mask) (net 3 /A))
  (pad 8 thru_hole oval (at 0 17.78) (size 1.7 1.7) (drill 1) (layers *.Cu *.Mask) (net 24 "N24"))
  (pad 9 thru_hole oval (at 0 20.32) (size 1.7 1.7) (drill 1) (layers *.Cu *.Mask) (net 26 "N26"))
  (pad 10 thru_hole oval (at 0 22.86) (size 1.7 1.7) (drill 1) (layers *.Cu *.Mask) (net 28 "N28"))
  (pad 11 thru_hole oval (at 0 25.4) (size 1.7 1.7) (drill 1) (layers *.Cu *.Mask) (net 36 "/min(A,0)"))
  (pad 13 thru_hole oval (at 0 30.48) (size 1.7 1.7) (drill 1) (layers *.Cu *.Mask) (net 10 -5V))
  (pad 14 thru_hole oval (at 0 33.02) (size 1.7 1.7) (drill 1) (layers *.Cu *.Mask) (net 2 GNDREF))
  (pad 15 thru_hole oval (at 0 35.56) (size 1.7 1.7) (drill 1) (layers *.Cu *.Mask) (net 9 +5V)))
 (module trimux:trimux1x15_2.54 (layer F.Cu) (at 62.5475 25.781)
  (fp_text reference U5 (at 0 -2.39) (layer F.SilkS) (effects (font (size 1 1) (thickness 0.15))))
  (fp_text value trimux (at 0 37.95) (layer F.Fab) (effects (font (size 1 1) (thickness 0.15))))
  (fp_line (start -1.39 1.27) (end -1.39 36.95) (layer F.SilkS) (width 0.12))
  (fp_line (start -1.39 36.95) (end 1.39 36.95) (layer F.SilkS) (width 0.12))
  (fp_line (start 1.39 36.95) (end 1.39 1.27) (layer F.SilkS) (width 0.12))
  (fp_line (start 1.39 1.27) (end -1.39 1.27) (layer F.SilkS) (width 0.12))
  (fp_line (start -1.39 0) (end -1.39 -1.39) (layer F.SilkS) (width 0.12))
  (fp_line (start -1.39 -1.39) (end 0 -1.39) (layer F.SilkS) (width 0.12))
  (pad 1 thru_hole rect (at 0 0) (size 1.7 1.7) (drill 1) (layers *.Cu *.Mask) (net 7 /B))
  (pad 2 thru_hole oval (at 0 2.54) (size 1.7 1.7) (drill 1) (layers *.Cu *.Mask) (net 33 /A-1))
  (pad 3 thru_hole oval (at 0 5.08) (size 1.7 1.7) (drill 1) (layers *.Cu *.Mask) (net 3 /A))
  (pad 4 thru_hole oval (at 0 7.62) (size 1.7 1.7) (drill 1) (layers *.Cu *.Mask) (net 34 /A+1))
  (pad 5 thru_hole oval (at 0 10.16) (size 1.7 1.7) (drill 1) (layers *.Cu *.Mask) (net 30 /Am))
  (pad 7 thru_hole oval (at 0 15.24) (size 1.7 1.7) (drill 1) (layers *.Cu *.Mask) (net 7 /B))
  (pad 8 thru_hole oval (at 0 17.78) (size 1.7 1.7) (drill 1) (layers *.Cu *.Mask) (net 36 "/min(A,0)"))
  (pad 9 thru_hole oval (at 0 20.32) (size 1.7 1.7) (drill 1) (layers *.Cu *.Mask) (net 29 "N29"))
  (pad 10 thru_hole oval (at 0 22.86) (size 1.7 1.7) (drill 1) (layers *.Cu *.Mask) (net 35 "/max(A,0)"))
  (pad 11 thru_hole oval (at 0 25.4) (size 1.7 1.7) (drill 1) (layers *.Cu *.Mask) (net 6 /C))
  (pad 13 thru_hole oval (at 0 30.48) (size 1.7 1.7) (drill 1) (layers *.Cu *.Mask) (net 10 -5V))
  (pad 14 thru_hole oval (at 0 33.02) (size 1.7 1.7) (drill 1) (layers *.Cu *.Mask) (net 2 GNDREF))
  (pad 15 thru_hole oval (at 0 35.56) (size 1.7 1.7) (drill 1) (layers *.Cu *.Mask) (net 9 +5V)))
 (gr_line (start 15 65) (end 15 15) (angle 90) (layer Edge.Cuts) (width 0.15))
 (gr_line (start 65 65) (end 15 65) (angle 90) (layer Edge.Cuts) (width 0.15))
 (gr_line (start 65 15) (end 65 65) (angle 90) (layer Edge.Cuts) (width 0.15))
 (gr_line (start 15 15) (end 65 15) (angle 90) (layer Edge.Cuts) (width 0.15))
 (segment (start 19.685 60.96) (end 24.384 60.96) (width 0.8) (layer F.Cu) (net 2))
 (segment (start 24.384 60.96) (end 29.21 60.96) (width 0.8) (layer F.Cu) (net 2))
 (segment (start 16.51 60.96) (end 19.685 60.96) (width 0.8) (layer B.Cu) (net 2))
 (segment (start 26.67 63.5) (end 26.67 57.245) (width 0.8) (layer B.Cu) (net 9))
 (segment (start 19.685 63.5) (end 26.67 63.5) (width 0.8) (layer B.Cu) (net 9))
 (segment (start 26.67 63.5) (end 29.21 63.5) (width 0.8) (layer B.Cu) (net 9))
 (segment (start 16.51 63.5) (end 19.685 63.5) (width 0.8) (layer B.Cu) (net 9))
 (segment (start 19.685 45.72) (end 19.78 45.72) (width 0.5) (layer B.Cu) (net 11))
 (segment (start 29.21 45.72) (end 29.115 45.72) (width 0.5) (layer B.Cu) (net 12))
 (segment (start 19.685 50.8) (end 19.78 50.8) (width 0.5) (layer B.Cu) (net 15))
 (segment (start 19.78 50.8) (end 22.225 53.245) (width 0.5) (layer B.Cu) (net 15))
 (segment (start 26.67 53.245) (end 26.765 53.245) (width 0.5) (layer B.Cu) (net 16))
 (segment (start 26.765 53.245) (end 29.21 50.8) (width 0.5) (layer B.Cu) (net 16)))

